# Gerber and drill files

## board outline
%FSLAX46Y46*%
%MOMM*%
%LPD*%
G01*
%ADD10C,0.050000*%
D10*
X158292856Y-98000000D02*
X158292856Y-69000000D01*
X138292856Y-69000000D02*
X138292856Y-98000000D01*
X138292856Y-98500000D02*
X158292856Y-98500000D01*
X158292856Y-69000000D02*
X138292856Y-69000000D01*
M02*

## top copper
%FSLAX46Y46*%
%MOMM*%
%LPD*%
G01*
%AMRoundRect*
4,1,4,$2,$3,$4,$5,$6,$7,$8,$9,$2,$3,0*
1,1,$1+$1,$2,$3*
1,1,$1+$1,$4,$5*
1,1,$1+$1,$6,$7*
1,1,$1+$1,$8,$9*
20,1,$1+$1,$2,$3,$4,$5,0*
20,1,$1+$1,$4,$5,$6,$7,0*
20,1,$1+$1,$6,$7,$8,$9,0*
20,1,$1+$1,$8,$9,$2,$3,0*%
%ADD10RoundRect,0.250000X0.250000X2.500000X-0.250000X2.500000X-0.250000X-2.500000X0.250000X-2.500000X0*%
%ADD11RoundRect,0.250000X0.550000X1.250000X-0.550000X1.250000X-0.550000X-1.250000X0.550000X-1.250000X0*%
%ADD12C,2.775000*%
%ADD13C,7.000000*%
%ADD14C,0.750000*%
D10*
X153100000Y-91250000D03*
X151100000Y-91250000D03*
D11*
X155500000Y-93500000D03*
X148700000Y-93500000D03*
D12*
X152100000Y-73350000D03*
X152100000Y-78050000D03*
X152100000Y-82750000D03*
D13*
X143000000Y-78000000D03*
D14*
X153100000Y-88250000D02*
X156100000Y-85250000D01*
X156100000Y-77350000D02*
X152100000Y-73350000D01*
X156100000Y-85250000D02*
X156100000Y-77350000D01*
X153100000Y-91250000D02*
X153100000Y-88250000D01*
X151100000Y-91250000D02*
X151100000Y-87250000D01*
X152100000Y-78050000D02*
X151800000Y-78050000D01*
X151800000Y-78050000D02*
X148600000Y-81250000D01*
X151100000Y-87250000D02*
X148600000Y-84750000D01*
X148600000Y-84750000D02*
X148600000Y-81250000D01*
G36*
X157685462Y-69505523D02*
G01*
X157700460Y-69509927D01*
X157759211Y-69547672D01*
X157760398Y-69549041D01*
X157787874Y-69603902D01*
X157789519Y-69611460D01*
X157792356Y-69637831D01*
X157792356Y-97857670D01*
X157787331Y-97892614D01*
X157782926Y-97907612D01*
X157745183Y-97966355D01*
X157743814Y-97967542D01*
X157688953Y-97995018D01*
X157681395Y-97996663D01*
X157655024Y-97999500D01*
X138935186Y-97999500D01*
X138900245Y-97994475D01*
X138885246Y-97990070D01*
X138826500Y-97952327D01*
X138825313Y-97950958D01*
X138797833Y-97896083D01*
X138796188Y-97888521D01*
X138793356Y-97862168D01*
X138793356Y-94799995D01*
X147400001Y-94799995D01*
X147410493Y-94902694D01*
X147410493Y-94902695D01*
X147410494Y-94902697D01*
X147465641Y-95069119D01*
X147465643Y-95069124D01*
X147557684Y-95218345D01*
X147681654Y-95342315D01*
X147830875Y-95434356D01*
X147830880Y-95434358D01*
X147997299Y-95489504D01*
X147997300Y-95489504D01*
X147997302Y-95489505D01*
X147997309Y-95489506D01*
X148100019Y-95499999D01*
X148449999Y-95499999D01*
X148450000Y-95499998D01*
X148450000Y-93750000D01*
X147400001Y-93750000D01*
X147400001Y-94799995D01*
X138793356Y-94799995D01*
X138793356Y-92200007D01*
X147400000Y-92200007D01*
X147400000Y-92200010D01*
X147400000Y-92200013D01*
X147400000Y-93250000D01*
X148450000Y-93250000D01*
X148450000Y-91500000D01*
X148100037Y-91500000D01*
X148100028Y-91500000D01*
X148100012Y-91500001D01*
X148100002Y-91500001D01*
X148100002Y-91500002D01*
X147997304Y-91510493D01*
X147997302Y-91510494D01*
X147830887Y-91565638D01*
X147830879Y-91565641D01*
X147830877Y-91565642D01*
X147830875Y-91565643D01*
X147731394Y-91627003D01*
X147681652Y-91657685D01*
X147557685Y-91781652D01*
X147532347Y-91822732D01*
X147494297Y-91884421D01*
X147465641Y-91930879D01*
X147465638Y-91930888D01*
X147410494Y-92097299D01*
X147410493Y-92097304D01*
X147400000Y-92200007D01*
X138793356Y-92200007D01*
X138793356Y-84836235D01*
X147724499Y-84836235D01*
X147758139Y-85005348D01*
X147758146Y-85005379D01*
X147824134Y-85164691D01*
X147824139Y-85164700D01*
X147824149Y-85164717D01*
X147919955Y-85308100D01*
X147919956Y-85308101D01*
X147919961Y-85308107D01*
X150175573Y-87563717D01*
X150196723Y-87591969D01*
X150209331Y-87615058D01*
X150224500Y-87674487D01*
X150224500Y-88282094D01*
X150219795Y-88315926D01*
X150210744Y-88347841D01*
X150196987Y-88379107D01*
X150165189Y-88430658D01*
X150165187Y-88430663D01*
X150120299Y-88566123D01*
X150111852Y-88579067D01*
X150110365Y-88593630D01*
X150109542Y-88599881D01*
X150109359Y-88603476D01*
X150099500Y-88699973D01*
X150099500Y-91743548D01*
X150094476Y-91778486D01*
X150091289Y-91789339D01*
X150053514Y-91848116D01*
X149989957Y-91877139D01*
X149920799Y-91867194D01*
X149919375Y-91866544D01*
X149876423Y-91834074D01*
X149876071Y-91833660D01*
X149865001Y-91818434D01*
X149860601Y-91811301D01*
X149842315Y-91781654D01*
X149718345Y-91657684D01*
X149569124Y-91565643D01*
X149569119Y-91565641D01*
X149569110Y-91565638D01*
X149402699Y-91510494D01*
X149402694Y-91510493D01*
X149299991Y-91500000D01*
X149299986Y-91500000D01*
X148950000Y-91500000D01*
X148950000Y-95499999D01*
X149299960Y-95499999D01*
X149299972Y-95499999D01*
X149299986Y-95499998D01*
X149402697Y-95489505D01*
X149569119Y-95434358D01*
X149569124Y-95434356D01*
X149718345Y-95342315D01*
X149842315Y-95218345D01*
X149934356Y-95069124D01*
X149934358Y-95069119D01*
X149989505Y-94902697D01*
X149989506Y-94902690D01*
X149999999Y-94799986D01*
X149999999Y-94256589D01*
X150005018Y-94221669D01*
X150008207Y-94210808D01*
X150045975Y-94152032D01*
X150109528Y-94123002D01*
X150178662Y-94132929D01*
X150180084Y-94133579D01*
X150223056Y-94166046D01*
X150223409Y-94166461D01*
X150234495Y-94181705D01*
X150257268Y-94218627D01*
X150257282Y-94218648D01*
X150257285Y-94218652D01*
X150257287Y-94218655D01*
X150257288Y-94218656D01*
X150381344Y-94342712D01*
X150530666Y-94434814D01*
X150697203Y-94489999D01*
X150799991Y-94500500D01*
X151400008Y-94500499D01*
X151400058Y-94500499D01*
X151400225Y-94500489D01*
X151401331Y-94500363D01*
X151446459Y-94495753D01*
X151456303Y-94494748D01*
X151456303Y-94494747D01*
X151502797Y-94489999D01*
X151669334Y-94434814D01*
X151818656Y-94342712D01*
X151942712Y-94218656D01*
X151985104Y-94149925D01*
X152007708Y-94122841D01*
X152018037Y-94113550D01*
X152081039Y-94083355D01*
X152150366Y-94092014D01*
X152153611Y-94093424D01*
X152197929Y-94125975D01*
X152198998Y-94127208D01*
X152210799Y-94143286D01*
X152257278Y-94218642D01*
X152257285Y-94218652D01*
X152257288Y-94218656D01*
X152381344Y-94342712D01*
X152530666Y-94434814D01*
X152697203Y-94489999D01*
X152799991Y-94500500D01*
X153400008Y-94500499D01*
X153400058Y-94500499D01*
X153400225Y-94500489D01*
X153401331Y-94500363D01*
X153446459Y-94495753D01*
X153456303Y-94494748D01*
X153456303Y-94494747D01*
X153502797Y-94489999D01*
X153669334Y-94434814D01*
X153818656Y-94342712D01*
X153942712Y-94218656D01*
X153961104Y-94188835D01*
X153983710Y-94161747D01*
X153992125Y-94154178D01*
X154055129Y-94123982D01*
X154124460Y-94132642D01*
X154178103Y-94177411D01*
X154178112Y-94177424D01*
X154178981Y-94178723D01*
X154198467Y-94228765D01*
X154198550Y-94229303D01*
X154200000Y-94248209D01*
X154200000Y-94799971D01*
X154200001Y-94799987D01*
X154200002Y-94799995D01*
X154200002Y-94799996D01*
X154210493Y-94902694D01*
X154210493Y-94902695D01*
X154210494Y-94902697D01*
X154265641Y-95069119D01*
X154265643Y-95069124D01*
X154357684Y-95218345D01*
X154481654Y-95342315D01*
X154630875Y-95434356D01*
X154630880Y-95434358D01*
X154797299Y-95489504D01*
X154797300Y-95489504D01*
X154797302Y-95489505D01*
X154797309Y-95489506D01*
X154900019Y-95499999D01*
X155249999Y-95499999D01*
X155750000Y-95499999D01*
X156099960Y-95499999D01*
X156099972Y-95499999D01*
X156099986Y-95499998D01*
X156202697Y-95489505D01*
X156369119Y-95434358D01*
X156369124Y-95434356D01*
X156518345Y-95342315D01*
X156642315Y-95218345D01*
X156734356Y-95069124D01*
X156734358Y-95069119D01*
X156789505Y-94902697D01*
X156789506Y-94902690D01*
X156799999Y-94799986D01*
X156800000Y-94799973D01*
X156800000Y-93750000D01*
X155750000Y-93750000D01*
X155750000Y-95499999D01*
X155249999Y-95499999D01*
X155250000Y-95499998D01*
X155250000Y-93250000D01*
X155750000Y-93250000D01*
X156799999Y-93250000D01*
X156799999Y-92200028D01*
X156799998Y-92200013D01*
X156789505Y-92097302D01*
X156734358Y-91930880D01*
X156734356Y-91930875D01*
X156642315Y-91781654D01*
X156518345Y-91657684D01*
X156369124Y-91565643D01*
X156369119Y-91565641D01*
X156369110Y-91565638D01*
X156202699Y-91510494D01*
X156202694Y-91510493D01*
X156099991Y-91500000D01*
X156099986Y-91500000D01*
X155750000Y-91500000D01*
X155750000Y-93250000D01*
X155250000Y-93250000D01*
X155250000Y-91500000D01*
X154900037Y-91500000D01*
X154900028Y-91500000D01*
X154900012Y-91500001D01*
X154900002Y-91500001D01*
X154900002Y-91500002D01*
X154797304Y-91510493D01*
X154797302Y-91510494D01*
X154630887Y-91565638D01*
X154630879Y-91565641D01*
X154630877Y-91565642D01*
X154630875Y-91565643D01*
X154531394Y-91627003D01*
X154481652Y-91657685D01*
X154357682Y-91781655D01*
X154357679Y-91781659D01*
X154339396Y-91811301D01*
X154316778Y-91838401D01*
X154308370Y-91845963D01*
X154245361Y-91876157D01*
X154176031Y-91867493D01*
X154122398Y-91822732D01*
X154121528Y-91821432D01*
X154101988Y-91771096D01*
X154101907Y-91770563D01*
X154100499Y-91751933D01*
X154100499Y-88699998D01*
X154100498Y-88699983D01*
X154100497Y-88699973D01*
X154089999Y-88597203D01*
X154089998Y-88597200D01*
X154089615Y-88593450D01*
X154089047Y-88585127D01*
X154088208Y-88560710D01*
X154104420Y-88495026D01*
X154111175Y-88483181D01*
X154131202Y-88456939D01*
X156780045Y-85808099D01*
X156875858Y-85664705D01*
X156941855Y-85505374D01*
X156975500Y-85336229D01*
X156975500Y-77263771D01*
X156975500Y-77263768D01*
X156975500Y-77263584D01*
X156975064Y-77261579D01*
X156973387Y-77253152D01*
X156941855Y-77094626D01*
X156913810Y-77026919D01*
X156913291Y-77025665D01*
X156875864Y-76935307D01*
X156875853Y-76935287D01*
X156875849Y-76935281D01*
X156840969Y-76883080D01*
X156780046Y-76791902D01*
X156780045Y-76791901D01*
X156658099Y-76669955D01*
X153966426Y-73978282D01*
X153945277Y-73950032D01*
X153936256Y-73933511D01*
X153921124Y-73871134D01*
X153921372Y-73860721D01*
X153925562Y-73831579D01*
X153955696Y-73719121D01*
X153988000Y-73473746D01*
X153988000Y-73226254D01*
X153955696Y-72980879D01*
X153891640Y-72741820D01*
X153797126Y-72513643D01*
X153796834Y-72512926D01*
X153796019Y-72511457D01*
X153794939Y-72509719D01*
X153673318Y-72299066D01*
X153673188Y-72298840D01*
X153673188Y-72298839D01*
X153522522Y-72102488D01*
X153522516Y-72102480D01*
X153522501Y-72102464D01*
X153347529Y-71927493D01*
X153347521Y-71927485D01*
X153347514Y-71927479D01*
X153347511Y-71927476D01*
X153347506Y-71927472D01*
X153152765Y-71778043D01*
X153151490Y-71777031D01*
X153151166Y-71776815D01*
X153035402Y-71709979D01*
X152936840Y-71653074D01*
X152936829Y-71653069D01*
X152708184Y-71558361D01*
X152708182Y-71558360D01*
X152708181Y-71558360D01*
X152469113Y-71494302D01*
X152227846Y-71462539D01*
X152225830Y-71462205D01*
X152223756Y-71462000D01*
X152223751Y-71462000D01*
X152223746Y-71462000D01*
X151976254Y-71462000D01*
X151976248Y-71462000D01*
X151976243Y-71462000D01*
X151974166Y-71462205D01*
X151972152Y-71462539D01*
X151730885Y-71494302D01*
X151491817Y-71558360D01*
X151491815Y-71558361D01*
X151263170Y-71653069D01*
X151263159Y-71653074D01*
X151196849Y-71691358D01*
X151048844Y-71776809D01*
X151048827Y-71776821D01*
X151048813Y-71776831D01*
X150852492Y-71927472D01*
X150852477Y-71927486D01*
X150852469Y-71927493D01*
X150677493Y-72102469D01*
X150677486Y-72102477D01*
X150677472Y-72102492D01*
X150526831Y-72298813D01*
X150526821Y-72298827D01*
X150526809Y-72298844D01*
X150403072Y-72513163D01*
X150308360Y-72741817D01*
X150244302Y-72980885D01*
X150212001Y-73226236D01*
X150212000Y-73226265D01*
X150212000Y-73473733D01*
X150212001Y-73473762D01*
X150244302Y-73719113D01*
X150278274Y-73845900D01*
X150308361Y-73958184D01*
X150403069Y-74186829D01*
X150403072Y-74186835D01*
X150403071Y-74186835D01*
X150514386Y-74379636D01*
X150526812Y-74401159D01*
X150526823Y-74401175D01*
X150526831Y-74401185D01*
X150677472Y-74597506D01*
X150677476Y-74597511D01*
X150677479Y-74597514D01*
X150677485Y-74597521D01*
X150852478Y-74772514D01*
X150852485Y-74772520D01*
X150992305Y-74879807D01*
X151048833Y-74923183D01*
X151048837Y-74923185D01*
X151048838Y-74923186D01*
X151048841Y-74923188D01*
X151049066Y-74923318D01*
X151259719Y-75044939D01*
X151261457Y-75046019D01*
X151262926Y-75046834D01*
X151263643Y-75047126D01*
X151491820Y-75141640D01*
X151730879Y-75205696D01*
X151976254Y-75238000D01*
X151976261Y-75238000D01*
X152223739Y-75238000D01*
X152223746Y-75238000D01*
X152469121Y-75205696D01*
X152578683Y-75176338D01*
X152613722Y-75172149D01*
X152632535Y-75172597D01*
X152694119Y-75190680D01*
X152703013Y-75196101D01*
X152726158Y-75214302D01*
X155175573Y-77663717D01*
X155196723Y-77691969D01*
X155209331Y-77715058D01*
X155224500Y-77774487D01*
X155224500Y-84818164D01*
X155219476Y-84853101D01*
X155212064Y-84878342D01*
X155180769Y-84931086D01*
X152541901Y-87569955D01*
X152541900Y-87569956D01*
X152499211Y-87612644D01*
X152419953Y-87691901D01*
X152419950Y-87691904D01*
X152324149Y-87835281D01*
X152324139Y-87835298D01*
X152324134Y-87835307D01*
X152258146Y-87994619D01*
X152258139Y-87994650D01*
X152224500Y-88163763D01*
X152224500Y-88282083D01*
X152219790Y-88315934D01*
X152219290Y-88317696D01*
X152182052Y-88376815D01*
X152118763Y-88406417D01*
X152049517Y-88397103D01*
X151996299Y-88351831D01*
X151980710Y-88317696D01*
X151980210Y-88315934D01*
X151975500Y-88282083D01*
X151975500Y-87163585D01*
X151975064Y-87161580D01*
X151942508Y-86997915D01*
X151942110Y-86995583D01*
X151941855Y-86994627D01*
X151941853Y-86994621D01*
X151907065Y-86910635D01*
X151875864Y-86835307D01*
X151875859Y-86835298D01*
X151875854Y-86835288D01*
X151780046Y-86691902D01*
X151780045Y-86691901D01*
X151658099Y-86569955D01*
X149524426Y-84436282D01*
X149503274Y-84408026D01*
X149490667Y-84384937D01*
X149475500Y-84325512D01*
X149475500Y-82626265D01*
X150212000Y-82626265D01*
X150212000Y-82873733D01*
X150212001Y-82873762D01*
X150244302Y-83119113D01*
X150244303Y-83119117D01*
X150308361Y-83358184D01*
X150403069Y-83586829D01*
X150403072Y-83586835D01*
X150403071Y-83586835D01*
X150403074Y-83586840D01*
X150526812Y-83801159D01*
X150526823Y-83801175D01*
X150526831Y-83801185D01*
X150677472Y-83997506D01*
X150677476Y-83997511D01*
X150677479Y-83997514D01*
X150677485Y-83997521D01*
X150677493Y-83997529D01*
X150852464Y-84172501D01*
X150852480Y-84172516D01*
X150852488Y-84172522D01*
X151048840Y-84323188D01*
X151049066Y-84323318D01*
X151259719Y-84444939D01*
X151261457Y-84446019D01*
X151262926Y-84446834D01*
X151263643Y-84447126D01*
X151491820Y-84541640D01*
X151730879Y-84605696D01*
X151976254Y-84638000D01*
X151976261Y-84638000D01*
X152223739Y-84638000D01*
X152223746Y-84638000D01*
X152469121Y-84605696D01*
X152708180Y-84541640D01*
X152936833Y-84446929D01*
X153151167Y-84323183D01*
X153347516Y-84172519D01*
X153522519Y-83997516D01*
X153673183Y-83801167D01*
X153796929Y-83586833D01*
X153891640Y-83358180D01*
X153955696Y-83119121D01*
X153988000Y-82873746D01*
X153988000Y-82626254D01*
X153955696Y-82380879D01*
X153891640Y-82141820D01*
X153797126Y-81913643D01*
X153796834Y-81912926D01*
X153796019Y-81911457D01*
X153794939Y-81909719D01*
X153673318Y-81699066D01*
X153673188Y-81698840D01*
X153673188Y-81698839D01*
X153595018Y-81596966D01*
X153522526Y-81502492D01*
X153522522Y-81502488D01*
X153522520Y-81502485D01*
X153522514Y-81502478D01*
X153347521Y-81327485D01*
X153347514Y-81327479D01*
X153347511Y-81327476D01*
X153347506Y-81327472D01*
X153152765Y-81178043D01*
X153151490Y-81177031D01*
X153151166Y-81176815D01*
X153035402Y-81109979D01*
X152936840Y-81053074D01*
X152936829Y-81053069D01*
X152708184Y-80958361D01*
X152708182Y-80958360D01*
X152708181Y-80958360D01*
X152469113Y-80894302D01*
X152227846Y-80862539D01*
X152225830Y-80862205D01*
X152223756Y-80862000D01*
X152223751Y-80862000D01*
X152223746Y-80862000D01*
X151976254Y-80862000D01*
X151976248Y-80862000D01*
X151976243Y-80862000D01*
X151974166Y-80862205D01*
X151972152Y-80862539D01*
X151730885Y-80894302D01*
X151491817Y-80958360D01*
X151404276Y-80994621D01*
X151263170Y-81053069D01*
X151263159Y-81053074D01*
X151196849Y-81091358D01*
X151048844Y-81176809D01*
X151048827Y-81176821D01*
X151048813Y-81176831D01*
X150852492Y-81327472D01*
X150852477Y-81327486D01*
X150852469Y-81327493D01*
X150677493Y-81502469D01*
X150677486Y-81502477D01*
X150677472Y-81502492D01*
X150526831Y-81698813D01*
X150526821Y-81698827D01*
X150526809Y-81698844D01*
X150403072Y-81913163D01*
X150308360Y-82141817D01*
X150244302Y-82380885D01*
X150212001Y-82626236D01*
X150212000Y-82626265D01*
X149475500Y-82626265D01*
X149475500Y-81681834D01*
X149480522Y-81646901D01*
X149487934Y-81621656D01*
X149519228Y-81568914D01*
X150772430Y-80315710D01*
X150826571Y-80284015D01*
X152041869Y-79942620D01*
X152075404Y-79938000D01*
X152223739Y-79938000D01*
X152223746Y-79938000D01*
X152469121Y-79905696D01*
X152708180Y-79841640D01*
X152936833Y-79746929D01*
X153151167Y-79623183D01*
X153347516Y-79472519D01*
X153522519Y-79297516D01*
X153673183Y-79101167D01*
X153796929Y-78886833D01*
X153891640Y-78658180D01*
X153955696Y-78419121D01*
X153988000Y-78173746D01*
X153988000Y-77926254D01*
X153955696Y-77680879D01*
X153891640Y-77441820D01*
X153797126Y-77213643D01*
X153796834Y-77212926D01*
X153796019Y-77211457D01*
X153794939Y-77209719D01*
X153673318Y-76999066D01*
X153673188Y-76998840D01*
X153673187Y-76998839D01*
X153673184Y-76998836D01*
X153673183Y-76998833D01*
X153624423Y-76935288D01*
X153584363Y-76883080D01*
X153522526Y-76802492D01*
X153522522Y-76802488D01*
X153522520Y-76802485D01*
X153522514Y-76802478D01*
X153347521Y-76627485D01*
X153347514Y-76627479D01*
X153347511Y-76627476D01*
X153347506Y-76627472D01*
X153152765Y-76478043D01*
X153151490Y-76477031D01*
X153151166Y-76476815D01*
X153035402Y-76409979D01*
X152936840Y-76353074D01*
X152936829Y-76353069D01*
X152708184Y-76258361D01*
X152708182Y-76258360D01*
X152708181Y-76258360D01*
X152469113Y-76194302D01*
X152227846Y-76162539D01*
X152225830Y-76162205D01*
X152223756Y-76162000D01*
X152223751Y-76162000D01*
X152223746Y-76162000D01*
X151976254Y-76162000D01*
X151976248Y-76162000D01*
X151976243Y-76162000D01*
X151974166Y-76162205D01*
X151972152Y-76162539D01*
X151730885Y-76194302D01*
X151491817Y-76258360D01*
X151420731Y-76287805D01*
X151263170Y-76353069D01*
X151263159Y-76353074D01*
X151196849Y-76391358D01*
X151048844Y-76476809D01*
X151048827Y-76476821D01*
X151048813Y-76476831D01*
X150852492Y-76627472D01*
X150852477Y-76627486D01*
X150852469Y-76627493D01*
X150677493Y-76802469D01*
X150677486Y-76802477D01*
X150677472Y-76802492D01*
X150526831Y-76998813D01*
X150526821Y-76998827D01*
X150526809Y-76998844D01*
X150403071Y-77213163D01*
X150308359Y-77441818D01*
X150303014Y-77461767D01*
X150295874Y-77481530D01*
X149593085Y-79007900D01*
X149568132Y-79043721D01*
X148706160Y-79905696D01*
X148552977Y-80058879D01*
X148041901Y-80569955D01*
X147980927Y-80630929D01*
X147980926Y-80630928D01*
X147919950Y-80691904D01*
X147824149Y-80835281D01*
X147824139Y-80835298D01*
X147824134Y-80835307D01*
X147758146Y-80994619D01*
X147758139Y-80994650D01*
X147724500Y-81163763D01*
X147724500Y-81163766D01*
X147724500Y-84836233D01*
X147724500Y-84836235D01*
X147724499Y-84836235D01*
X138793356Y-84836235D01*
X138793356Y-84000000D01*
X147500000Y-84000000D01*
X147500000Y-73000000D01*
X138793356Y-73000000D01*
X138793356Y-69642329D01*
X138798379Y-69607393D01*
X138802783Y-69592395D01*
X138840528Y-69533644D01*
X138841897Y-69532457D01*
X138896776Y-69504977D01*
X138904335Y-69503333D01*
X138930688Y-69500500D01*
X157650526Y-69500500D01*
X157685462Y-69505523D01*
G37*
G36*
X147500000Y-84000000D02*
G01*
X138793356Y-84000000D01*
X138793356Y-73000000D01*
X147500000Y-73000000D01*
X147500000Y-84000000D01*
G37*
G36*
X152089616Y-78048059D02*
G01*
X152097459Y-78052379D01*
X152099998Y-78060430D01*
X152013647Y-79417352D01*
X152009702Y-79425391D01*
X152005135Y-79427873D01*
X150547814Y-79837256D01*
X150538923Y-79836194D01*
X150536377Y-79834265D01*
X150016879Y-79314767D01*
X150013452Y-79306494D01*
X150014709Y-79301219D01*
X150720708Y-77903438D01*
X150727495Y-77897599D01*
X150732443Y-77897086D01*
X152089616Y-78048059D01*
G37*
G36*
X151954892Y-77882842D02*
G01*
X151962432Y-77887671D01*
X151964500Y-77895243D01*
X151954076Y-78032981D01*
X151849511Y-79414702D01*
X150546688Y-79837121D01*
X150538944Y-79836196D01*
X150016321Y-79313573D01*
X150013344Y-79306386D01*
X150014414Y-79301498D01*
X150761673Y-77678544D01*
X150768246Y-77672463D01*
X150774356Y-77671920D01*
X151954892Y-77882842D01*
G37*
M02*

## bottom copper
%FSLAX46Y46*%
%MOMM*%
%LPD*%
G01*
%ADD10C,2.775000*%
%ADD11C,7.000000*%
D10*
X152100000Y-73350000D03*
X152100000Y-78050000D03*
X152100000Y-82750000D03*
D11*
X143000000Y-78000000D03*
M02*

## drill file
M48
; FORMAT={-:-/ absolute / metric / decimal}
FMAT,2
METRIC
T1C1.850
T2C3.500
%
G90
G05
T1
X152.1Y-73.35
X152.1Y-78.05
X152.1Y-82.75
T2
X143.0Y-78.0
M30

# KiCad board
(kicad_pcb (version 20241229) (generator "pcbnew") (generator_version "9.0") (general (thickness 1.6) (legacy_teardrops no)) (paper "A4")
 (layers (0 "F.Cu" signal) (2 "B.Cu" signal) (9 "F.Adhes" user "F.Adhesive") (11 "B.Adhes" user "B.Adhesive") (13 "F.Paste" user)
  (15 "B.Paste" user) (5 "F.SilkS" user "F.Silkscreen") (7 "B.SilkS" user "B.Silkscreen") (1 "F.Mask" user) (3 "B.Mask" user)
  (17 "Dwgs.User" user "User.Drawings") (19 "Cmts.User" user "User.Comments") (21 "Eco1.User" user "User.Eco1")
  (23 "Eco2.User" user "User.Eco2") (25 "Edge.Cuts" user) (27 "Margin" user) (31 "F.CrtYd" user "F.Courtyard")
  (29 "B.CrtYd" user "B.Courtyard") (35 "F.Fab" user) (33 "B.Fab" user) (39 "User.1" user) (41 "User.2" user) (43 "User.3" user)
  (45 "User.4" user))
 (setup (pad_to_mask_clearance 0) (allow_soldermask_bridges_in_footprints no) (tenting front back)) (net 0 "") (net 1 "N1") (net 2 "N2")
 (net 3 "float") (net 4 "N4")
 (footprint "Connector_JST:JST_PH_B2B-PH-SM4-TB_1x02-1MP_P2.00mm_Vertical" (layer "F.Cu") (at 152.1 91.75 180)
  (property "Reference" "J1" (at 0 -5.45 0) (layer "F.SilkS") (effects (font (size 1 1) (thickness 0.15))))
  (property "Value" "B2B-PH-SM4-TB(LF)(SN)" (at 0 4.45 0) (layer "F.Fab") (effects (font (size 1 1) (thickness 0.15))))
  (pad "1" smd roundrect (at -1 0.5 180) (size 1 5.5) (layers "F.Cu" "F.Mask" "F.Paste") (roundrect_rratio 0.25) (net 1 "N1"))
  (pad "2" smd roundrect (at 1 0.5 180) (size 1 5.5) (layers "F.Cu" "F.Mask" "F.Paste") (roundrect_rratio 0.25) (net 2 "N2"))
  (pad "MP" smd roundrect (at -3.4 -1.75 180) (size 1.6 3) (layers "F.Cu" "F.Mask" "F.Paste") (roundrect_rratio 0.15625) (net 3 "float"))
  (pad "MP" smd roundrect (at 3.4 -1.75 180) (size 1.6 3) (layers "F.Cu" "F.Mask" "F.Paste") (roundrect_rratio 0.15625) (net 3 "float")))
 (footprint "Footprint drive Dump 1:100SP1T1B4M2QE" (layer "B.Cu") (at 152.1 78.05 -90)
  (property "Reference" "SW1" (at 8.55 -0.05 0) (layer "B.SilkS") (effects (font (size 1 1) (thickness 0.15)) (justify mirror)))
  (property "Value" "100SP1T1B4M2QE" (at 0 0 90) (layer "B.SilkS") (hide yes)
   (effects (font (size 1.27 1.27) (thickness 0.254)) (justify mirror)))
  (pad "1" thru_hole circle (at -4.7 0 270) (size 2.775 2.775) (drill 1.85) (layers "*.Cu" "*.Mask") (remove_unused_layers no) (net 1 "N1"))
  (pad "2" thru_hole circle (at 0 0 270) (size 2.775 2.775) (drill 1.85) (layers "*.Cu" "*.Mask") (remove_unused_layers no) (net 2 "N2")
   (teardrops (best_length_ratio 0.5) (max_length 1) (best_width_ratio 1) (max_width 2) (curved_edges no) (filter_ratio 0.9) (enabled yes)
    (allow_two_segments yes) (prefer_zone_connections yes)))
  (pad "3" thru_hole circle (at 4.7 0 270) (size 2.775 2.775) (drill 1.85) (layers "*.Cu" "*.Mask") (remove_unused_layers no) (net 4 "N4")
   (teardrops (best_length_ratio 0.5) (max_length 1) (best_width_ratio 1) (max_width 2) (curved_edges no) (filter_ratio 0.9) (enabled yes)
    (allow_two_segments yes) (prefer_zone_connections yes))))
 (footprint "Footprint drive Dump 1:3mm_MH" (layer "B.Cu") (at 143 78 180)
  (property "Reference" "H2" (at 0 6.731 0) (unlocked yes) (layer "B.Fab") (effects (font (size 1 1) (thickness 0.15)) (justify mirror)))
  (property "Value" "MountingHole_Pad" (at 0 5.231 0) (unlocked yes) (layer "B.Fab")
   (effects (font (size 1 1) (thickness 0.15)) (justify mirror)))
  (pad "1" thru_hole circle (at 0 0 180) (size 7 7) (drill 3.5) (layers "*.Cu" "*.Mask") (remove_unused_layers no) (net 3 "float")))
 (gr_line (start 158.292856 98) (end 158.292856 69) (stroke (width 0.05) (type default)) (layer "Edge.Cuts"))
 (gr_line (start 138.292856 69) (end 138.292856 98) (stroke (width 0.05) (type default)) (layer "Edge.Cuts"))
 (gr_line (start 138.292856 98.5) (end 158.292856 98.5) (stroke (width 0.05) (type default)) (layer "Edge.Cuts"))
 (gr_line (start 158.292856 69) (end 138.292856 69) (stroke (width 0.05) (type default)) (layer "Edge.Cuts"))
 (segment (start 153.1 88.25) (end 156.1 85.25) (width 0.75) (layer "F.Cu") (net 1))
 (segment (start 156.1 77.35) (end 152.1 73.35) (width 0.75) (layer "F.Cu") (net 1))
 (segment (start 156.1 85.25) (end 156.1 77.35) (width 0.75) (layer "F.Cu") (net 1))
 (segment (start 153.1 91.25) (end 153.1 88.25) (width 0.75) (layer "F.Cu") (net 1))
 (segment (start 151.1 91.25) (end 151.1 87.25) (width 0.75) (layer "F.Cu") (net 2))
 (segment (start 152.1 78.05) (end 151.8 78.05) (width 0.75) (layer "F.Cu") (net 2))
 (segment (start 151.8 78.05) (end 148.6 81.25) (width 0.75) (layer "F.Cu") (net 2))
 (segment (start 151.1 87.25) (end 148.6 84.75) (width 0.75) (layer "F.Cu") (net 2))
 (segment (start 148.6 84.75) (end 148.6 81.25) (width 0.75) (layer "F.Cu") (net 2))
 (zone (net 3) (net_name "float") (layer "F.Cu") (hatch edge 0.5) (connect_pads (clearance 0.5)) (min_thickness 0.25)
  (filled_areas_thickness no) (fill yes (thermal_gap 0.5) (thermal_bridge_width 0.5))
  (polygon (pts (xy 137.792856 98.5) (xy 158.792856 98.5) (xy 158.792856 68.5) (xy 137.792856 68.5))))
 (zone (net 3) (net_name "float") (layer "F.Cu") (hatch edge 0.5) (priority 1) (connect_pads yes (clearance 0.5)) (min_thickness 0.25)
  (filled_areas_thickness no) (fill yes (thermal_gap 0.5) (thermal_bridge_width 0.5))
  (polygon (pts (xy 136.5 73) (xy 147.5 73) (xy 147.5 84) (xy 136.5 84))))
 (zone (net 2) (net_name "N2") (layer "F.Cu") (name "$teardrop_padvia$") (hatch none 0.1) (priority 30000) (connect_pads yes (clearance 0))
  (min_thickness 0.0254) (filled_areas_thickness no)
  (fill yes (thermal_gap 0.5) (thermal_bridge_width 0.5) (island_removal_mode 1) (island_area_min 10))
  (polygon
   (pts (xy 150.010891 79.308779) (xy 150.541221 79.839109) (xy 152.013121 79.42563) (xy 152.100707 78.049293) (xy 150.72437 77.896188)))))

